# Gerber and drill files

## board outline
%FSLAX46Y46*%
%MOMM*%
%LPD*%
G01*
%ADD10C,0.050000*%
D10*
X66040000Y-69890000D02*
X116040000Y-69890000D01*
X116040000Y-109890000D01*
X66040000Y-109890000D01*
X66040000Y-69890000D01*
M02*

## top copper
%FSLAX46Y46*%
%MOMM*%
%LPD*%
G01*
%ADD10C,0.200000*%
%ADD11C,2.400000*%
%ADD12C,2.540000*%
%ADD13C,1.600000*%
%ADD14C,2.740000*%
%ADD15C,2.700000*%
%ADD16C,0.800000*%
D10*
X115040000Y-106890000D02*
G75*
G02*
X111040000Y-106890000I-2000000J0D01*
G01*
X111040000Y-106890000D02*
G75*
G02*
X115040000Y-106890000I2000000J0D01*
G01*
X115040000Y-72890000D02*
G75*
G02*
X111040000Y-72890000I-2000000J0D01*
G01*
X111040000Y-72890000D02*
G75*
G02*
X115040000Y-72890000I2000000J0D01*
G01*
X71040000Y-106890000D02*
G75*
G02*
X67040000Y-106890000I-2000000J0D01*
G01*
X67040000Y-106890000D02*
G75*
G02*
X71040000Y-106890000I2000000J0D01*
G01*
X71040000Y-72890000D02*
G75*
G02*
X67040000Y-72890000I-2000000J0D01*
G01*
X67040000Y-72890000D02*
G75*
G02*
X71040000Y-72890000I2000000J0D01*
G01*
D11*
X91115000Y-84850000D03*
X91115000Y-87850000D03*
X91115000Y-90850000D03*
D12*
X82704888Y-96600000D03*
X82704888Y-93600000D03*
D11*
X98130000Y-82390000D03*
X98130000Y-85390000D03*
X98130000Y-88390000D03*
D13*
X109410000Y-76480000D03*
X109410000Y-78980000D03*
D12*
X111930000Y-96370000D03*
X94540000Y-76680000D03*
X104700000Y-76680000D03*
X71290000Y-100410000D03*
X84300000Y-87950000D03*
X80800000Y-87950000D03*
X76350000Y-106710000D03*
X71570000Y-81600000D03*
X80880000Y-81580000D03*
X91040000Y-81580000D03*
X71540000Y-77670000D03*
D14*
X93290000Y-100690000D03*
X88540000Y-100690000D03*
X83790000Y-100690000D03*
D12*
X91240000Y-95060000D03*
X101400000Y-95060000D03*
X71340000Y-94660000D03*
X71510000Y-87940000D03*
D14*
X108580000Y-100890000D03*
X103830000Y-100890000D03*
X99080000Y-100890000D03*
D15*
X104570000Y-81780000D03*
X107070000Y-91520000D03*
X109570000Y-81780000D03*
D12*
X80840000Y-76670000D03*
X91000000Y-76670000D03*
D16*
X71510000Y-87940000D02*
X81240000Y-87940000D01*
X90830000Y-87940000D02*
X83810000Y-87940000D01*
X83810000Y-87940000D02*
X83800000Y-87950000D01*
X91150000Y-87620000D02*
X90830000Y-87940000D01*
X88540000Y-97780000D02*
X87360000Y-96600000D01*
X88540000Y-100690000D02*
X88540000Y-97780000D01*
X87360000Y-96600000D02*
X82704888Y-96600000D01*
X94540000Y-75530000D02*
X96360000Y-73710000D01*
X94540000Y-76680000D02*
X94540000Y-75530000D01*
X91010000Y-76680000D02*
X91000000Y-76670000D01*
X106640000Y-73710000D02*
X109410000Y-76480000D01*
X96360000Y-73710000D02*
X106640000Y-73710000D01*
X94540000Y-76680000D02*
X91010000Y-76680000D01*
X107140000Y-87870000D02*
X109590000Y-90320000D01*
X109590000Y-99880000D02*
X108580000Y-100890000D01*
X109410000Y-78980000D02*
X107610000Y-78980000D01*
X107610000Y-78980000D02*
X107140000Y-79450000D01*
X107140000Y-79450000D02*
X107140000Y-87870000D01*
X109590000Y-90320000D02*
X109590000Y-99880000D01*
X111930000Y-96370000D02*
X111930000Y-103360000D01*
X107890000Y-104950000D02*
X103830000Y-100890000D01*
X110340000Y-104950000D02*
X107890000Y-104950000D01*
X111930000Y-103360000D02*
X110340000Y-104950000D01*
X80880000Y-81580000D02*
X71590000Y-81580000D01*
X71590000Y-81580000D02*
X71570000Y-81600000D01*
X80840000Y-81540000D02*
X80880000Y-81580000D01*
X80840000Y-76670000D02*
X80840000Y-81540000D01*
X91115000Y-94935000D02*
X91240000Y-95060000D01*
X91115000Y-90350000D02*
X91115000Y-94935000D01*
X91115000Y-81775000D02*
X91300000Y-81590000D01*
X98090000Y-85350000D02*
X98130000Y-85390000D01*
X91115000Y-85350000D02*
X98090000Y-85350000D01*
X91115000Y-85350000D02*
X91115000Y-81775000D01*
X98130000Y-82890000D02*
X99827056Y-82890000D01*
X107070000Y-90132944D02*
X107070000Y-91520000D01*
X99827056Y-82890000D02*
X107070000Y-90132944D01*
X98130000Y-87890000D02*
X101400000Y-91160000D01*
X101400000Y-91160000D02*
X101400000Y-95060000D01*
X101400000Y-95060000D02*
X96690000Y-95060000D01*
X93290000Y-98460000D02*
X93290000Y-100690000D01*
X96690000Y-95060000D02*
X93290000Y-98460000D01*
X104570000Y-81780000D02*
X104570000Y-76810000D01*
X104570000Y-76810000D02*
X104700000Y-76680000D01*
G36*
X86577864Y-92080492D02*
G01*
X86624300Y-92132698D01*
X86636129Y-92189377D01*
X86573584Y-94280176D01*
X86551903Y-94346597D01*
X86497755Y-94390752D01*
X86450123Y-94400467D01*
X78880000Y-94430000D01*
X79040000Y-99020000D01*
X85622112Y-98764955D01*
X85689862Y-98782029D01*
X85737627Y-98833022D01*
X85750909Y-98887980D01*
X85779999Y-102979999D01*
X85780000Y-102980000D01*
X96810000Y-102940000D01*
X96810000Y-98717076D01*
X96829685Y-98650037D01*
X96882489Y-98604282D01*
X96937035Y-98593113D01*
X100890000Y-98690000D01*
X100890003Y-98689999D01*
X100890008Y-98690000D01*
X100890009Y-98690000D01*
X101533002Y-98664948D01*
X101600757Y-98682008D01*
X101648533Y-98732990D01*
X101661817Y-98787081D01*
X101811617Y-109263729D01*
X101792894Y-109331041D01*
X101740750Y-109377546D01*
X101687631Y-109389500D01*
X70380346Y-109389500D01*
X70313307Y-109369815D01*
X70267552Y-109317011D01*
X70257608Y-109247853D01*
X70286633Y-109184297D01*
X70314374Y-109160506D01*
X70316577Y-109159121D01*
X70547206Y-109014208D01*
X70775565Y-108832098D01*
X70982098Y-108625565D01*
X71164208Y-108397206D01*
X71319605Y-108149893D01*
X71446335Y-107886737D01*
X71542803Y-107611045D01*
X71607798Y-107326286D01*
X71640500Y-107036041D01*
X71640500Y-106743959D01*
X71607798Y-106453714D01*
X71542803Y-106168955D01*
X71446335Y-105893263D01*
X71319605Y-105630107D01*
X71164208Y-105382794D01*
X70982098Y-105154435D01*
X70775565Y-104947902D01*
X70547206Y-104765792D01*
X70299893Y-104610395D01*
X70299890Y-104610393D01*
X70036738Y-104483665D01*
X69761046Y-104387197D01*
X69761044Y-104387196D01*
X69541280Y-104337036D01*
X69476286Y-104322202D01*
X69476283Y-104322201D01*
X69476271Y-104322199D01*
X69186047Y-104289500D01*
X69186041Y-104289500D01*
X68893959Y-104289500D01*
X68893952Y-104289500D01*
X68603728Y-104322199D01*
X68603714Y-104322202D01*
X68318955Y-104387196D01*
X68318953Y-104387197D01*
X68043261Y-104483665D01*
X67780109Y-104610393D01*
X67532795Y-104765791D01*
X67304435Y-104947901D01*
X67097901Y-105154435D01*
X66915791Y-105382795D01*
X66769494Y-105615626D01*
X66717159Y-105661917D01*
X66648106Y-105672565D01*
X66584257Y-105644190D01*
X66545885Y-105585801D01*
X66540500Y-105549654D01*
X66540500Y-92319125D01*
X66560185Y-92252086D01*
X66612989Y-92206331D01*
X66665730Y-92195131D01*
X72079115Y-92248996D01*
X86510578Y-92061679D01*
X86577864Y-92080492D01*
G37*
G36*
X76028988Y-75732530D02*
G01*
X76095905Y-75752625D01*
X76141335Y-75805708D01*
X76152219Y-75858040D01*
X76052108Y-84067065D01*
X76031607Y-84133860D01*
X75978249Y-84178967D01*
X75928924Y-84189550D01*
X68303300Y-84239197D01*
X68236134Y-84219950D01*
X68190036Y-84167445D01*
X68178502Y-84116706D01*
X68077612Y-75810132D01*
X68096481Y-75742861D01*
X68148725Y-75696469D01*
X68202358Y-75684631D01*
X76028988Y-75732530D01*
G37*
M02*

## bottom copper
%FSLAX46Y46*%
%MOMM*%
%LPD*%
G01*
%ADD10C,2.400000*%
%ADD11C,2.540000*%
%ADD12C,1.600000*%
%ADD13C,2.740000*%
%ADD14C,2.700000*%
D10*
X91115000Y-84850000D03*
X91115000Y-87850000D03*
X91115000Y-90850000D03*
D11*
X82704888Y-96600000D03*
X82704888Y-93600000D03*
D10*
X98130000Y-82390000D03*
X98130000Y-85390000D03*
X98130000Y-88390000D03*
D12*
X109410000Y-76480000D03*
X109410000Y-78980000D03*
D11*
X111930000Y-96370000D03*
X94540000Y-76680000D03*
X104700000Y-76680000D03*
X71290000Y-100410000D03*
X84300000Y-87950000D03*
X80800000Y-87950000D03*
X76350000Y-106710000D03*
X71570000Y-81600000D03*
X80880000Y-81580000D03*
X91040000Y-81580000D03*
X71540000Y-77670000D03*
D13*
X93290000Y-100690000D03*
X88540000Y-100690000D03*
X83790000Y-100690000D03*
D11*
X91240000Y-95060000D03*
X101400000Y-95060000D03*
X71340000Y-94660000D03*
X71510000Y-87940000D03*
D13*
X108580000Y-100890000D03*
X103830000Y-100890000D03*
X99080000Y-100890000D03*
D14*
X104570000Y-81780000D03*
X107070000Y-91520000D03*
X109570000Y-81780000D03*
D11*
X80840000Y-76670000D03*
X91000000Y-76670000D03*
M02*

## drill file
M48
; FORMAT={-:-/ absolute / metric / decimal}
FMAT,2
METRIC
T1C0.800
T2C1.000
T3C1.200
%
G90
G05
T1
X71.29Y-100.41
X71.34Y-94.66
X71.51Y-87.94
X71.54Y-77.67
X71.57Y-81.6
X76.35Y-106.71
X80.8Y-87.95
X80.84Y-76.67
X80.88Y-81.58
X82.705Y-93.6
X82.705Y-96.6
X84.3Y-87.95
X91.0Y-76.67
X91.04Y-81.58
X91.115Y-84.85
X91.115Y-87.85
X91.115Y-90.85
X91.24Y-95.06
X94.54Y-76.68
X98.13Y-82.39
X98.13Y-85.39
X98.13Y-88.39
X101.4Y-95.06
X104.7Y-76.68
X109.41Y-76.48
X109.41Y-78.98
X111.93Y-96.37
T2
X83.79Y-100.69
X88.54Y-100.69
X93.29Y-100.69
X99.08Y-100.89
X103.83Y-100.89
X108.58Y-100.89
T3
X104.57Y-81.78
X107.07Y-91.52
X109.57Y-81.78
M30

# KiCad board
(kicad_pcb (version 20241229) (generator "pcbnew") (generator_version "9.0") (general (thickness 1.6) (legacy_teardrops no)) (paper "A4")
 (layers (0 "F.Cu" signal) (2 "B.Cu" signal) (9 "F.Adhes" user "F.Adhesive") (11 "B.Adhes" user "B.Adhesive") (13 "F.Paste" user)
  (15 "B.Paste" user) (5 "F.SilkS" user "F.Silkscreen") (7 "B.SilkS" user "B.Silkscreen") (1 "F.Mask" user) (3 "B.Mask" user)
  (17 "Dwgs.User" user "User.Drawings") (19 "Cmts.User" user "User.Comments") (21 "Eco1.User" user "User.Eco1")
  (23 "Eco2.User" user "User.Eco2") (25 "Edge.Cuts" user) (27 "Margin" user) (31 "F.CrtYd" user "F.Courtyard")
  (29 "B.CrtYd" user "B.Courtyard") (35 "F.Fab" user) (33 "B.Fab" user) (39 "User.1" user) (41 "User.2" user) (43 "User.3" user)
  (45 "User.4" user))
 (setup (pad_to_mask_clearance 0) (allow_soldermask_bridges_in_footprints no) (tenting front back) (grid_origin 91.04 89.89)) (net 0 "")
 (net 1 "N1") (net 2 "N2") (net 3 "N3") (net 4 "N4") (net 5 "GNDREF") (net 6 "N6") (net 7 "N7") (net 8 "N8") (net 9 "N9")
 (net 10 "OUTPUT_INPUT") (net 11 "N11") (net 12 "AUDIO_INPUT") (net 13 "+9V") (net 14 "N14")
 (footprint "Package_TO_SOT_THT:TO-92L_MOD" (layer "F.Cu") (at 91.115 86.85 -90)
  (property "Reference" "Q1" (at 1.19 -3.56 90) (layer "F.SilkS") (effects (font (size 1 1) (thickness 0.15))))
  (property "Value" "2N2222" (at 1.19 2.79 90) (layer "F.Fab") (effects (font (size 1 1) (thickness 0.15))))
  (pad "1" thru_hole circle (at -2 0 270) (size 2.4 2.4) (drill 0.8) (layers "*.Cu" "*.Mask") (remove_unused_layers no) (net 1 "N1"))
  (pad "2" thru_hole circle (at 1 0 270) (size 2.4 2.4) (drill 0.8) (layers "*.Cu" "*.Mask") (remove_unused_layers no) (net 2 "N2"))
  (pad "3" thru_hole circle (at 4 0 270) (size 2.4 2.4) (drill 0.8) (layers "*.Cu" "*.Mask") (remove_unused_layers no) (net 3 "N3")))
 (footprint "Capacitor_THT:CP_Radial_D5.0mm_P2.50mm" (layer "F.Cu") (at 82.704888 96.1 90)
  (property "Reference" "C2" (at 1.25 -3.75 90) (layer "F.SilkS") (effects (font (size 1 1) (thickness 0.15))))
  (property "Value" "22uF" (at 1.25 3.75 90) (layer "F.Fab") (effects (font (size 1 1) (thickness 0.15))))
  (pad "1" thru_hole circle (at -0.5 0 90) (size 2.54 2.54) (drill 0.8) (layers "*.Cu" "*.Mask") (remove_unused_layers no) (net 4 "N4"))
  (pad "2" thru_hole circle (at 2.5 0 90) (size 2.54 2.54) (drill 0.8) (layers "*.Cu" "*.Mask") (remove_unused_layers no) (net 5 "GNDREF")))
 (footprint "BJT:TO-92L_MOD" (layer "F.Cu") (at 98.13 84.39 -90)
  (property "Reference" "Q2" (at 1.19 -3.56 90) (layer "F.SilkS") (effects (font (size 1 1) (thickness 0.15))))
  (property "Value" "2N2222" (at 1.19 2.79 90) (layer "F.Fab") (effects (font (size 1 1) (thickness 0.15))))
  (pad "1" thru_hole circle (at -2 0 270) (size 2.4 2.4) (drill 0.8) (layers "*.Cu" "*.Mask") (remove_unused_layers no) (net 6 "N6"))
  (pad "2" thru_hole circle (at 1 0 270) (size 2.4 2.4) (drill 0.8) (layers "*.Cu" "*.Mask") (remove_unused_layers no) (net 1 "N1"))
  (pad "3" thru_hole circle (at 4 0 270) (size 2.4 2.4) (drill 0.8) (layers "*.Cu" "*.Mask") (remove_unused_layers no) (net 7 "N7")))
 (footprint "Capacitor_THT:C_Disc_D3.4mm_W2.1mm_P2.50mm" (layer "F.Cu") (at 109.41 76.48 -90)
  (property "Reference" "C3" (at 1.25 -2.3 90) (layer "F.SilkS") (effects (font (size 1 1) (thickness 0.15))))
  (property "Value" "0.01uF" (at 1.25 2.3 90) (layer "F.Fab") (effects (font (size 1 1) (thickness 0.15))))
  (pad "1" thru_hole circle (at 0 0 270) (size 1.6 1.6) (drill 0.8) (layers "*.Cu" "*.Mask") (remove_unused_layers no) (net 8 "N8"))
  (pad "2" thru_hole circle (at 2.5 0 270) (size 1.6 1.6) (drill 0.8) (layers "*.Cu" "*.Mask") (remove_unused_layers no) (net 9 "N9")))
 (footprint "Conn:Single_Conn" (layer "F.Cu") (at 111.93 98.87)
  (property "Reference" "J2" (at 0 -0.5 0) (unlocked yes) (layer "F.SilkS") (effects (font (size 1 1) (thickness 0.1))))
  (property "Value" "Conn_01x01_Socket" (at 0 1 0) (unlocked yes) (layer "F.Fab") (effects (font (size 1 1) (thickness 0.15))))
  (pad "1" thru_hole circle (at 0 -2.5) (size 2.54 2.54) (drill 0.8) (layers "*.Cu" "*.Mask") (remove_unused_layers no)
   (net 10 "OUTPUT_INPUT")))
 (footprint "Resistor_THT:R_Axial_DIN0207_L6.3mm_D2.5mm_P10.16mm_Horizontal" (layer "F.Cu") (at 94.54 76.68)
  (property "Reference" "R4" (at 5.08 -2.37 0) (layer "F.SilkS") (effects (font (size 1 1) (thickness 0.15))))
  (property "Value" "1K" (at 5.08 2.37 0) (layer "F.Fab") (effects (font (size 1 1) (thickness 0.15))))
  (pad "1" thru_hole circle (at 0 0) (size 2.54 2.54) (drill 0.8) (layers "*.Cu" "*.Mask") (remove_unused_layers no) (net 8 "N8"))
  (pad "2" thru_hole circle (at 10.16 0) (size 2.54 2.54) (drill 0.8) (layers "*.Cu" "*.Mask") (remove_unused_layers no) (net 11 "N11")))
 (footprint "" (layer "F.Cu") (at 71.29 100.41)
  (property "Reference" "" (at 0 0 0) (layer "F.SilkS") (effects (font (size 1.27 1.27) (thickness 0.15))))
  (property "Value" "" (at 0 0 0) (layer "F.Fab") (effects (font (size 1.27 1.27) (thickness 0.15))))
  (pad "1" thru_hole circle (at 0 0 90) (size 2.54 2.54) (drill 0.8) (layers "*.Cu" "*.Mask") (remove_unused_layers no) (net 5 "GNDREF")))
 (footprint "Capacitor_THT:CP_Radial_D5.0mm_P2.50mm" (layer "F.Cu") (at 83.8 87.95 180)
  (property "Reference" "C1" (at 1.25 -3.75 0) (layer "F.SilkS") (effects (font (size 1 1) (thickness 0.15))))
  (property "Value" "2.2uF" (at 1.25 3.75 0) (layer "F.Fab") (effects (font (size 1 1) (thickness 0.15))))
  (pad "1" thru_hole circle (at -0.5 0 180) (size 2.54 2.54) (drill 0.8) (layers "*.Cu" "*.Mask") (remove_unused_layers no) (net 2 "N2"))
  (pad "2" thru_hole circle (at 3 0 180) (size 2.54 2.54) (drill 0.8) (layers "*.Cu" "*.Mask") (remove_unused_layers no)
   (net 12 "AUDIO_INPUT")))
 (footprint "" (layer "F.Cu") (at 76.35 106.71)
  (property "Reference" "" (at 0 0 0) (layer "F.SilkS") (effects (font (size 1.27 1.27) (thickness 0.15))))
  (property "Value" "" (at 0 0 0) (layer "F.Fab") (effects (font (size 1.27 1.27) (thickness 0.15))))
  (pad "1" thru_hole circle (at 0 0 90) (size 2.54 2.54) (drill 0.8) (layers "*.Cu" "*.Mask") (remove_unused_layers no) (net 5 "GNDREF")))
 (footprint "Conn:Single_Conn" (layer "F.Cu") (at 69.07 81.6 -90)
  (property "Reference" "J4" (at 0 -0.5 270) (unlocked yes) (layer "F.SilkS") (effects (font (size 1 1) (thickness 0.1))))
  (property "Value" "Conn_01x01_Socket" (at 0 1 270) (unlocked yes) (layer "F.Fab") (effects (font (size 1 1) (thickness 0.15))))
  (pad "1" thru_hole circle (at 0 -2.5 270) (size 2.54 2.54) (drill 0.8) (layers "*.Cu" "*.Mask") (remove_unused_layers no) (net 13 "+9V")))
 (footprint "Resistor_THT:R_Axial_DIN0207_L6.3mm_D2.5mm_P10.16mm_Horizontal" (layer "F.Cu") (at 80.88 81.58)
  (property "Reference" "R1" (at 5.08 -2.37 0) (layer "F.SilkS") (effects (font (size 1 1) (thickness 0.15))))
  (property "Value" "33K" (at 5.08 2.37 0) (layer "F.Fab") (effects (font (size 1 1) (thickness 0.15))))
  (pad "1" thru_hole circle (at 0 0) (size 2.54 2.54) (drill 0.8) (layers "*.Cu" "*.Mask") (remove_unused_layers no) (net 13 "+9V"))
  (pad "2" thru_hole circle (at 10.16 0) (size 2.54 2.54) (drill 0.8) (layers "*.Cu" "*.Mask") (remove_unused_layers no) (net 1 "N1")))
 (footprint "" (layer "F.Cu") (at 71.54 77.67)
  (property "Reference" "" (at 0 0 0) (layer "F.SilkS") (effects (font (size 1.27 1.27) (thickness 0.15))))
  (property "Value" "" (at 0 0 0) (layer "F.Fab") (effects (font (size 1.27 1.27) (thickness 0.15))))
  (pad "1" thru_hole circle (at 0 0 270) (size 2.54 2.54) (drill 0.8) (layers "*.Cu" "*.Mask") (remove_unused_layers no) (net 13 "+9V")))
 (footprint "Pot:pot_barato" (layer "F.Cu") (at 88.54 100.69 90)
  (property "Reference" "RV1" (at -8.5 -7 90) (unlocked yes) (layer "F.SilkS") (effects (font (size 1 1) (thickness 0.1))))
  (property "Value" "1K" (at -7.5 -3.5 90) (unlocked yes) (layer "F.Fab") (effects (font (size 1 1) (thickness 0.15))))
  (pad "1" thru_hole circle (at 0 4.75 90) (size 2.74 2.74) (drill 1) (layers "*.Cu" "*.Mask") (remove_unused_layers no) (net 7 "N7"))
  (pad "2" thru_hole circle (at 0 0 90) (size 2.74 2.74) (drill 1) (layers "*.Cu" "*.Mask") (remove_unused_layers no) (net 4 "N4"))
  (pad "3" thru_hole circle (at 0 -4.75 90) (size 2.74 2.74) (drill 1) (layers "*.Cu" "*.Mask") (remove_unused_layers no) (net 5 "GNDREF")))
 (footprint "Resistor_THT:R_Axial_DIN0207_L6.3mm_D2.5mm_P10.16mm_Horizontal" (layer "F.Cu") (at 91.24 95.06)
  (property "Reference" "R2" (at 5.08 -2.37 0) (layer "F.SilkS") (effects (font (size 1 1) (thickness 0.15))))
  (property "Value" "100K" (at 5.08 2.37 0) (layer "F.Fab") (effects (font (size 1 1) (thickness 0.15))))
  (pad "1" thru_hole circle (at 0 0) (size 2.54 2.54) (drill 0.8) (layers "*.Cu" "*.Mask") (remove_unused_layers no) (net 3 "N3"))
  (pad "2" thru_hole circle (at 10.16 0) (size 2.54 2.54) (drill 0.8) (layers "*.Cu" "*.Mask") (remove_unused_layers no) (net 7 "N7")))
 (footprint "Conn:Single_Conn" (layer "F.Cu") (at 73.84 94.66 90)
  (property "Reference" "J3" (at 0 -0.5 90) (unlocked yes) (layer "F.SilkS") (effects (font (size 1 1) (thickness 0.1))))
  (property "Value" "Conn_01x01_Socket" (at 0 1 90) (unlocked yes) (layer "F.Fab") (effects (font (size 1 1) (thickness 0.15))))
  (pad "1" thru_hole circle (at 0 -2.5 90) (size 2.54 2.54) (drill 0.8) (layers "*.Cu" "*.Mask") (remove_unused_layers no) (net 5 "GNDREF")))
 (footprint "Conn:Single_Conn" (layer "F.Cu") (at 74.01 87.94 90)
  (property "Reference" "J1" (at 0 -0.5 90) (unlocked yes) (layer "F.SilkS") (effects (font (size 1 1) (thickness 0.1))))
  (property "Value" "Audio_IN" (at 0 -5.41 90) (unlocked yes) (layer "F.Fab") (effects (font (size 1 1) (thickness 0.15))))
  (pad "1" thru_hole circle (at 0 -2.5 90) (size 2.54 2.54) (drill 0.8) (layers "*.Cu" "*.Mask") (remove_unused_layers no)
   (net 12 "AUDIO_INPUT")))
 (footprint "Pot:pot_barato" (layer "F.Cu") (at 103.83 100.89 90)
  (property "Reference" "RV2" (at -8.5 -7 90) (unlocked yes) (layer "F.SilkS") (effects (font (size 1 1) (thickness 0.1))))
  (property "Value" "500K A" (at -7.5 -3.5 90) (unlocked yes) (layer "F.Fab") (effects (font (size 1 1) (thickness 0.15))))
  (pad "1" thru_hole circle (at 0 4.75 90) (size 2.74 2.74) (drill 1) (layers "*.Cu" "*.Mask") (remove_unused_layers no) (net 9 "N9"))
  (pad "2" thru_hole circle (at 0 0 90) (size 2.74 2.74) (drill 1) (layers "*.Cu" "*.Mask") (remove_unused_layers no)
   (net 10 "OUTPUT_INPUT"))
  (pad "3" thru_hole circle (at 0 -4.75 90) (size 2.74 2.74) (drill 1) (layers "*.Cu" "*.Mask") (remove_unused_layers no) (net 5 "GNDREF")))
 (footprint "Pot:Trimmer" (layer "F.Cu") (at 107.07 81.78 180)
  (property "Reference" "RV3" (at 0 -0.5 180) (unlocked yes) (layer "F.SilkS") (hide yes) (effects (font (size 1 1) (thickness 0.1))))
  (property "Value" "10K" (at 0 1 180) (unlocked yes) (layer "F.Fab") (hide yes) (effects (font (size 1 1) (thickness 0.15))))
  (pad "1" thru_hole circle (at 2.5 0 180) (size 2.7 2.7) (drill 1.2) (layers "*.Cu" "*.Mask") (remove_unused_layers no) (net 11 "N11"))
  (pad "2" thru_hole circle (at 0 -9.74 180) (size 2.7 2.7) (drill 1.2) (layers "*.Cu" "*.Mask") (remove_unused_layers no) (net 6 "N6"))
  (pad "3" thru_hole circle (at -2.5 0 180) (size 2.7 2.7) (drill 1.2) (layers "*.Cu" "*.Mask") (remove_unused_layers no) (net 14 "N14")))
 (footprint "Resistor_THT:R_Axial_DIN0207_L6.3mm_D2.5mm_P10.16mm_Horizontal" (layer "F.Cu") (at 80.84 76.67)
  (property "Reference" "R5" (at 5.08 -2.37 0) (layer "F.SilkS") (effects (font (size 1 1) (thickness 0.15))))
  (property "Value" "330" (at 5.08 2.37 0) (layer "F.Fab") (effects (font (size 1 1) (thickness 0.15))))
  (pad "1" thru_hole circle (at 0 0) (size 2.54 2.54) (drill 0.8) (layers "*.Cu" "*.Mask") (remove_unused_layers no) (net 13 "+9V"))
  (pad "2" thru_hole circle (at 10.16 0) (size 2.54 2.54) (drill 0.8) (layers "*.Cu" "*.Mask") (remove_unused_layers no) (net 8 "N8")))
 (gr_circle (center 113.04 106.89) (end 115.04 106.89) (stroke (width 0.2) (type solid)) (fill no) (layer "F.Cu"))
 (gr_circle (center 113.04 72.89) (end 115.04 72.89) (stroke (width 0.2) (type solid)) (fill no) (layer "F.Cu"))
 (gr_circle (center 69.04 106.89) (end 71.04 106.89) (stroke (width 0.2) (type solid)) (fill no) (layer "F.Cu"))
 (gr_circle (center 69.04 72.89) (end 71.04 72.89) (stroke (width 0.2) (type solid)) (fill no) (layer "F.Cu"))
 (gr_rect (start 66.04 69.89) (end 116.04 109.89) (stroke (width 0.05) (type solid)) (fill no) (layer "Edge.Cuts"))
 (segment (start 71.51 87.94) (end 81.24 87.94) (width 0.8) (layer "F.Cu") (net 12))
 (segment (start 90.83 87.94) (end 83.81 87.94) (width 0.8) (layer "F.Cu") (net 2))
 (segment (start 83.81 87.94) (end 83.8 87.95) (width 0.8) (layer "F.Cu") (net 2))
 (segment (start 91.15 87.62) (end 90.83 87.94) (width 0.8) (layer "F.Cu") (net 2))
 (segment (start 88.54 97.78) (end 87.36 96.6) (width 0.8) (layer "F.Cu") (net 4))
 (segment (start 88.54 100.69) (end 88.54 97.78) (width 0.8) (layer "F.Cu") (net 4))
 (segment (start 87.36 96.6) (end 82.704888 96.6) (width 0.8) (layer "F.Cu") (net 4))
 (segment (start 94.54 75.53) (end 96.36 73.71) (width 0.8) (layer "F.Cu") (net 8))
 (segment (start 94.54 76.68) (end 94.54 75.53) (width 0.8) (layer "F.Cu") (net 8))
 (segment (start 91.01 76.68) (end 91 76.67) (width 0.8) (layer "F.Cu") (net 8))
 (segment (start 106.64 73.71) (end 109.41 76.48) (width 0.8) (layer "F.Cu") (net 8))
 (segment (start 96.36 73.71) (end 106.64 73.71) (width 0.8) (layer "F.Cu") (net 8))
 (segment (start 94.54 76.68) (end 91.01 76.68) (width 0.8) (layer "F.Cu") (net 8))
 (segment (start 107.14 87.87) (end 109.59 90.32) (width 0.8) (layer "F.Cu") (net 9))
 (segment (start 109.59 99.88) (end 108.58 100.89) (width 0.8) (layer "F.Cu") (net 9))
 (segment (start 109.41 78.98) (end 107.61 78.98) (width 0.8) (layer "F.Cu") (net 9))
 (segment (start 107.61 78.98) (end 107.14 79.45) (width 0.8) (layer "F.Cu") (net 9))
 (segment (start 107.14 79.45) (end 107.14 87.87) (width 0.8) (layer "F.Cu") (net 9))
 (segment (start 109.59 90.32) (end 109.59 99.88) (width 0.8) (layer "F.Cu") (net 9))
 (segment (start 111.93 96.37) (end 111.93 103.36) (width 0.8) (layer "F.Cu") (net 10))
 (segment (start 107.89 104.95) (end 103.83 100.89) (width 0.8) (layer "F.Cu") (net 10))
 (segment (start 110.34 104.95) (end 107.89 104.95) (width 0.8) (layer "F.Cu") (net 10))
 (segment (start 111.93 103.36) (end 110.34 104.95) (width 0.8) (layer "F.Cu") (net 10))
 (segment (start 80.88 81.58) (end 71.59 81.58) (width 0.8) (layer "F.Cu") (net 13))
 (segment (start 71.59 81.58) (end 71.57 81.6) (width 0.8) (layer "F.Cu") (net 13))
 (segment (start 80.84 81.54) (end 80.88 81.58) (width 0.8) (layer "F.Cu") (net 13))
 (segment (start 80.84 76.67) (end 80.84 81.54) (width 0.8) (layer "F.Cu") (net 13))
 (segment (start 91.115 94.935) (end 91.24 95.06) (width 0.8) (layer "F.Cu") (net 3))
 (segment (start 91.115 90.35) (end 91.115 94.935) (width 0.8) (layer "F.Cu") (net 3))
 (segment (start 91.115 81.775) (end 91.3 81.59) (width 0.8) (layer "F.Cu") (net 1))
 (segment (start 98.09 85.35) (end 98.13 85.39) (width 0.8) (layer "F.Cu") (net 1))
 (segment (start 91.115 85.35) (end 98.09 85.35) (width 0.8) (layer "F.Cu") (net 1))
 (segment (start 91.115 85.35) (end 91.115 81.775) (width 0.8) (layer "F.Cu") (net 1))
 (segment (start 98.13 82.89) (end 99.827056 82.89) (width 0.8) (layer "F.Cu") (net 6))
 (segment (start 107.07 90.132944) (end 107.07 91.52) (width 0.8) (layer "F.Cu") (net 6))
 (segment (start 99.827056 82.89) (end 107.07 90.132944) (width 0.8) (layer "F.Cu") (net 6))
 (segment (start 98.13 87.89) (end 101.4 91.16) (width 0.8) (layer "F.Cu") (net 7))
 (segment (start 101.4 91.16) (end 101.4 95.06) (width 0.8) (layer "F.Cu") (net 7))
 (segment (start 101.4 95.06) (end 96.69 95.06) (width 0.8) (layer "F.Cu") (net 7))
 (segment (start 93.29 98.46) (end 93.29 100.69) (width 0.8) (layer "F.Cu") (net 7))
 (segment (start 96.69 95.06) (end 93.29 98.46) (width 0.8) (layer "F.Cu") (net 7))
 (segment (start 104.57 81.78) (end 104.57 76.81) (width 0.8) (layer "F.Cu") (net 11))
 (segment (start 104.57 76.81) (end 104.7 76.68) (width 0.8) (layer "F.Cu") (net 11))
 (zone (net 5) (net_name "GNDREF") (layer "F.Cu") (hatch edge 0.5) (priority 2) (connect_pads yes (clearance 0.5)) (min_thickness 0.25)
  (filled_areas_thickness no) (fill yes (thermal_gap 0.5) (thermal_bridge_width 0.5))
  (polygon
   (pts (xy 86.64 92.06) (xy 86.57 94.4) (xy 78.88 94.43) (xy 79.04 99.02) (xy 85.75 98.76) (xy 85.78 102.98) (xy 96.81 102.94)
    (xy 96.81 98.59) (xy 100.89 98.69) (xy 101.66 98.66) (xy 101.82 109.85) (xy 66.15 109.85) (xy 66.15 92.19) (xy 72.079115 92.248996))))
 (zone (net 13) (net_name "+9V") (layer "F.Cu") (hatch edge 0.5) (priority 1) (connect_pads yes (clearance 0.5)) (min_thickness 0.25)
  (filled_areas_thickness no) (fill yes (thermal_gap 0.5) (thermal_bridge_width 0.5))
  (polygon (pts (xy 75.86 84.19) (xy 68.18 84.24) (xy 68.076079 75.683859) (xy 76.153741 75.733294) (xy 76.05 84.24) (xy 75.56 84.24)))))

